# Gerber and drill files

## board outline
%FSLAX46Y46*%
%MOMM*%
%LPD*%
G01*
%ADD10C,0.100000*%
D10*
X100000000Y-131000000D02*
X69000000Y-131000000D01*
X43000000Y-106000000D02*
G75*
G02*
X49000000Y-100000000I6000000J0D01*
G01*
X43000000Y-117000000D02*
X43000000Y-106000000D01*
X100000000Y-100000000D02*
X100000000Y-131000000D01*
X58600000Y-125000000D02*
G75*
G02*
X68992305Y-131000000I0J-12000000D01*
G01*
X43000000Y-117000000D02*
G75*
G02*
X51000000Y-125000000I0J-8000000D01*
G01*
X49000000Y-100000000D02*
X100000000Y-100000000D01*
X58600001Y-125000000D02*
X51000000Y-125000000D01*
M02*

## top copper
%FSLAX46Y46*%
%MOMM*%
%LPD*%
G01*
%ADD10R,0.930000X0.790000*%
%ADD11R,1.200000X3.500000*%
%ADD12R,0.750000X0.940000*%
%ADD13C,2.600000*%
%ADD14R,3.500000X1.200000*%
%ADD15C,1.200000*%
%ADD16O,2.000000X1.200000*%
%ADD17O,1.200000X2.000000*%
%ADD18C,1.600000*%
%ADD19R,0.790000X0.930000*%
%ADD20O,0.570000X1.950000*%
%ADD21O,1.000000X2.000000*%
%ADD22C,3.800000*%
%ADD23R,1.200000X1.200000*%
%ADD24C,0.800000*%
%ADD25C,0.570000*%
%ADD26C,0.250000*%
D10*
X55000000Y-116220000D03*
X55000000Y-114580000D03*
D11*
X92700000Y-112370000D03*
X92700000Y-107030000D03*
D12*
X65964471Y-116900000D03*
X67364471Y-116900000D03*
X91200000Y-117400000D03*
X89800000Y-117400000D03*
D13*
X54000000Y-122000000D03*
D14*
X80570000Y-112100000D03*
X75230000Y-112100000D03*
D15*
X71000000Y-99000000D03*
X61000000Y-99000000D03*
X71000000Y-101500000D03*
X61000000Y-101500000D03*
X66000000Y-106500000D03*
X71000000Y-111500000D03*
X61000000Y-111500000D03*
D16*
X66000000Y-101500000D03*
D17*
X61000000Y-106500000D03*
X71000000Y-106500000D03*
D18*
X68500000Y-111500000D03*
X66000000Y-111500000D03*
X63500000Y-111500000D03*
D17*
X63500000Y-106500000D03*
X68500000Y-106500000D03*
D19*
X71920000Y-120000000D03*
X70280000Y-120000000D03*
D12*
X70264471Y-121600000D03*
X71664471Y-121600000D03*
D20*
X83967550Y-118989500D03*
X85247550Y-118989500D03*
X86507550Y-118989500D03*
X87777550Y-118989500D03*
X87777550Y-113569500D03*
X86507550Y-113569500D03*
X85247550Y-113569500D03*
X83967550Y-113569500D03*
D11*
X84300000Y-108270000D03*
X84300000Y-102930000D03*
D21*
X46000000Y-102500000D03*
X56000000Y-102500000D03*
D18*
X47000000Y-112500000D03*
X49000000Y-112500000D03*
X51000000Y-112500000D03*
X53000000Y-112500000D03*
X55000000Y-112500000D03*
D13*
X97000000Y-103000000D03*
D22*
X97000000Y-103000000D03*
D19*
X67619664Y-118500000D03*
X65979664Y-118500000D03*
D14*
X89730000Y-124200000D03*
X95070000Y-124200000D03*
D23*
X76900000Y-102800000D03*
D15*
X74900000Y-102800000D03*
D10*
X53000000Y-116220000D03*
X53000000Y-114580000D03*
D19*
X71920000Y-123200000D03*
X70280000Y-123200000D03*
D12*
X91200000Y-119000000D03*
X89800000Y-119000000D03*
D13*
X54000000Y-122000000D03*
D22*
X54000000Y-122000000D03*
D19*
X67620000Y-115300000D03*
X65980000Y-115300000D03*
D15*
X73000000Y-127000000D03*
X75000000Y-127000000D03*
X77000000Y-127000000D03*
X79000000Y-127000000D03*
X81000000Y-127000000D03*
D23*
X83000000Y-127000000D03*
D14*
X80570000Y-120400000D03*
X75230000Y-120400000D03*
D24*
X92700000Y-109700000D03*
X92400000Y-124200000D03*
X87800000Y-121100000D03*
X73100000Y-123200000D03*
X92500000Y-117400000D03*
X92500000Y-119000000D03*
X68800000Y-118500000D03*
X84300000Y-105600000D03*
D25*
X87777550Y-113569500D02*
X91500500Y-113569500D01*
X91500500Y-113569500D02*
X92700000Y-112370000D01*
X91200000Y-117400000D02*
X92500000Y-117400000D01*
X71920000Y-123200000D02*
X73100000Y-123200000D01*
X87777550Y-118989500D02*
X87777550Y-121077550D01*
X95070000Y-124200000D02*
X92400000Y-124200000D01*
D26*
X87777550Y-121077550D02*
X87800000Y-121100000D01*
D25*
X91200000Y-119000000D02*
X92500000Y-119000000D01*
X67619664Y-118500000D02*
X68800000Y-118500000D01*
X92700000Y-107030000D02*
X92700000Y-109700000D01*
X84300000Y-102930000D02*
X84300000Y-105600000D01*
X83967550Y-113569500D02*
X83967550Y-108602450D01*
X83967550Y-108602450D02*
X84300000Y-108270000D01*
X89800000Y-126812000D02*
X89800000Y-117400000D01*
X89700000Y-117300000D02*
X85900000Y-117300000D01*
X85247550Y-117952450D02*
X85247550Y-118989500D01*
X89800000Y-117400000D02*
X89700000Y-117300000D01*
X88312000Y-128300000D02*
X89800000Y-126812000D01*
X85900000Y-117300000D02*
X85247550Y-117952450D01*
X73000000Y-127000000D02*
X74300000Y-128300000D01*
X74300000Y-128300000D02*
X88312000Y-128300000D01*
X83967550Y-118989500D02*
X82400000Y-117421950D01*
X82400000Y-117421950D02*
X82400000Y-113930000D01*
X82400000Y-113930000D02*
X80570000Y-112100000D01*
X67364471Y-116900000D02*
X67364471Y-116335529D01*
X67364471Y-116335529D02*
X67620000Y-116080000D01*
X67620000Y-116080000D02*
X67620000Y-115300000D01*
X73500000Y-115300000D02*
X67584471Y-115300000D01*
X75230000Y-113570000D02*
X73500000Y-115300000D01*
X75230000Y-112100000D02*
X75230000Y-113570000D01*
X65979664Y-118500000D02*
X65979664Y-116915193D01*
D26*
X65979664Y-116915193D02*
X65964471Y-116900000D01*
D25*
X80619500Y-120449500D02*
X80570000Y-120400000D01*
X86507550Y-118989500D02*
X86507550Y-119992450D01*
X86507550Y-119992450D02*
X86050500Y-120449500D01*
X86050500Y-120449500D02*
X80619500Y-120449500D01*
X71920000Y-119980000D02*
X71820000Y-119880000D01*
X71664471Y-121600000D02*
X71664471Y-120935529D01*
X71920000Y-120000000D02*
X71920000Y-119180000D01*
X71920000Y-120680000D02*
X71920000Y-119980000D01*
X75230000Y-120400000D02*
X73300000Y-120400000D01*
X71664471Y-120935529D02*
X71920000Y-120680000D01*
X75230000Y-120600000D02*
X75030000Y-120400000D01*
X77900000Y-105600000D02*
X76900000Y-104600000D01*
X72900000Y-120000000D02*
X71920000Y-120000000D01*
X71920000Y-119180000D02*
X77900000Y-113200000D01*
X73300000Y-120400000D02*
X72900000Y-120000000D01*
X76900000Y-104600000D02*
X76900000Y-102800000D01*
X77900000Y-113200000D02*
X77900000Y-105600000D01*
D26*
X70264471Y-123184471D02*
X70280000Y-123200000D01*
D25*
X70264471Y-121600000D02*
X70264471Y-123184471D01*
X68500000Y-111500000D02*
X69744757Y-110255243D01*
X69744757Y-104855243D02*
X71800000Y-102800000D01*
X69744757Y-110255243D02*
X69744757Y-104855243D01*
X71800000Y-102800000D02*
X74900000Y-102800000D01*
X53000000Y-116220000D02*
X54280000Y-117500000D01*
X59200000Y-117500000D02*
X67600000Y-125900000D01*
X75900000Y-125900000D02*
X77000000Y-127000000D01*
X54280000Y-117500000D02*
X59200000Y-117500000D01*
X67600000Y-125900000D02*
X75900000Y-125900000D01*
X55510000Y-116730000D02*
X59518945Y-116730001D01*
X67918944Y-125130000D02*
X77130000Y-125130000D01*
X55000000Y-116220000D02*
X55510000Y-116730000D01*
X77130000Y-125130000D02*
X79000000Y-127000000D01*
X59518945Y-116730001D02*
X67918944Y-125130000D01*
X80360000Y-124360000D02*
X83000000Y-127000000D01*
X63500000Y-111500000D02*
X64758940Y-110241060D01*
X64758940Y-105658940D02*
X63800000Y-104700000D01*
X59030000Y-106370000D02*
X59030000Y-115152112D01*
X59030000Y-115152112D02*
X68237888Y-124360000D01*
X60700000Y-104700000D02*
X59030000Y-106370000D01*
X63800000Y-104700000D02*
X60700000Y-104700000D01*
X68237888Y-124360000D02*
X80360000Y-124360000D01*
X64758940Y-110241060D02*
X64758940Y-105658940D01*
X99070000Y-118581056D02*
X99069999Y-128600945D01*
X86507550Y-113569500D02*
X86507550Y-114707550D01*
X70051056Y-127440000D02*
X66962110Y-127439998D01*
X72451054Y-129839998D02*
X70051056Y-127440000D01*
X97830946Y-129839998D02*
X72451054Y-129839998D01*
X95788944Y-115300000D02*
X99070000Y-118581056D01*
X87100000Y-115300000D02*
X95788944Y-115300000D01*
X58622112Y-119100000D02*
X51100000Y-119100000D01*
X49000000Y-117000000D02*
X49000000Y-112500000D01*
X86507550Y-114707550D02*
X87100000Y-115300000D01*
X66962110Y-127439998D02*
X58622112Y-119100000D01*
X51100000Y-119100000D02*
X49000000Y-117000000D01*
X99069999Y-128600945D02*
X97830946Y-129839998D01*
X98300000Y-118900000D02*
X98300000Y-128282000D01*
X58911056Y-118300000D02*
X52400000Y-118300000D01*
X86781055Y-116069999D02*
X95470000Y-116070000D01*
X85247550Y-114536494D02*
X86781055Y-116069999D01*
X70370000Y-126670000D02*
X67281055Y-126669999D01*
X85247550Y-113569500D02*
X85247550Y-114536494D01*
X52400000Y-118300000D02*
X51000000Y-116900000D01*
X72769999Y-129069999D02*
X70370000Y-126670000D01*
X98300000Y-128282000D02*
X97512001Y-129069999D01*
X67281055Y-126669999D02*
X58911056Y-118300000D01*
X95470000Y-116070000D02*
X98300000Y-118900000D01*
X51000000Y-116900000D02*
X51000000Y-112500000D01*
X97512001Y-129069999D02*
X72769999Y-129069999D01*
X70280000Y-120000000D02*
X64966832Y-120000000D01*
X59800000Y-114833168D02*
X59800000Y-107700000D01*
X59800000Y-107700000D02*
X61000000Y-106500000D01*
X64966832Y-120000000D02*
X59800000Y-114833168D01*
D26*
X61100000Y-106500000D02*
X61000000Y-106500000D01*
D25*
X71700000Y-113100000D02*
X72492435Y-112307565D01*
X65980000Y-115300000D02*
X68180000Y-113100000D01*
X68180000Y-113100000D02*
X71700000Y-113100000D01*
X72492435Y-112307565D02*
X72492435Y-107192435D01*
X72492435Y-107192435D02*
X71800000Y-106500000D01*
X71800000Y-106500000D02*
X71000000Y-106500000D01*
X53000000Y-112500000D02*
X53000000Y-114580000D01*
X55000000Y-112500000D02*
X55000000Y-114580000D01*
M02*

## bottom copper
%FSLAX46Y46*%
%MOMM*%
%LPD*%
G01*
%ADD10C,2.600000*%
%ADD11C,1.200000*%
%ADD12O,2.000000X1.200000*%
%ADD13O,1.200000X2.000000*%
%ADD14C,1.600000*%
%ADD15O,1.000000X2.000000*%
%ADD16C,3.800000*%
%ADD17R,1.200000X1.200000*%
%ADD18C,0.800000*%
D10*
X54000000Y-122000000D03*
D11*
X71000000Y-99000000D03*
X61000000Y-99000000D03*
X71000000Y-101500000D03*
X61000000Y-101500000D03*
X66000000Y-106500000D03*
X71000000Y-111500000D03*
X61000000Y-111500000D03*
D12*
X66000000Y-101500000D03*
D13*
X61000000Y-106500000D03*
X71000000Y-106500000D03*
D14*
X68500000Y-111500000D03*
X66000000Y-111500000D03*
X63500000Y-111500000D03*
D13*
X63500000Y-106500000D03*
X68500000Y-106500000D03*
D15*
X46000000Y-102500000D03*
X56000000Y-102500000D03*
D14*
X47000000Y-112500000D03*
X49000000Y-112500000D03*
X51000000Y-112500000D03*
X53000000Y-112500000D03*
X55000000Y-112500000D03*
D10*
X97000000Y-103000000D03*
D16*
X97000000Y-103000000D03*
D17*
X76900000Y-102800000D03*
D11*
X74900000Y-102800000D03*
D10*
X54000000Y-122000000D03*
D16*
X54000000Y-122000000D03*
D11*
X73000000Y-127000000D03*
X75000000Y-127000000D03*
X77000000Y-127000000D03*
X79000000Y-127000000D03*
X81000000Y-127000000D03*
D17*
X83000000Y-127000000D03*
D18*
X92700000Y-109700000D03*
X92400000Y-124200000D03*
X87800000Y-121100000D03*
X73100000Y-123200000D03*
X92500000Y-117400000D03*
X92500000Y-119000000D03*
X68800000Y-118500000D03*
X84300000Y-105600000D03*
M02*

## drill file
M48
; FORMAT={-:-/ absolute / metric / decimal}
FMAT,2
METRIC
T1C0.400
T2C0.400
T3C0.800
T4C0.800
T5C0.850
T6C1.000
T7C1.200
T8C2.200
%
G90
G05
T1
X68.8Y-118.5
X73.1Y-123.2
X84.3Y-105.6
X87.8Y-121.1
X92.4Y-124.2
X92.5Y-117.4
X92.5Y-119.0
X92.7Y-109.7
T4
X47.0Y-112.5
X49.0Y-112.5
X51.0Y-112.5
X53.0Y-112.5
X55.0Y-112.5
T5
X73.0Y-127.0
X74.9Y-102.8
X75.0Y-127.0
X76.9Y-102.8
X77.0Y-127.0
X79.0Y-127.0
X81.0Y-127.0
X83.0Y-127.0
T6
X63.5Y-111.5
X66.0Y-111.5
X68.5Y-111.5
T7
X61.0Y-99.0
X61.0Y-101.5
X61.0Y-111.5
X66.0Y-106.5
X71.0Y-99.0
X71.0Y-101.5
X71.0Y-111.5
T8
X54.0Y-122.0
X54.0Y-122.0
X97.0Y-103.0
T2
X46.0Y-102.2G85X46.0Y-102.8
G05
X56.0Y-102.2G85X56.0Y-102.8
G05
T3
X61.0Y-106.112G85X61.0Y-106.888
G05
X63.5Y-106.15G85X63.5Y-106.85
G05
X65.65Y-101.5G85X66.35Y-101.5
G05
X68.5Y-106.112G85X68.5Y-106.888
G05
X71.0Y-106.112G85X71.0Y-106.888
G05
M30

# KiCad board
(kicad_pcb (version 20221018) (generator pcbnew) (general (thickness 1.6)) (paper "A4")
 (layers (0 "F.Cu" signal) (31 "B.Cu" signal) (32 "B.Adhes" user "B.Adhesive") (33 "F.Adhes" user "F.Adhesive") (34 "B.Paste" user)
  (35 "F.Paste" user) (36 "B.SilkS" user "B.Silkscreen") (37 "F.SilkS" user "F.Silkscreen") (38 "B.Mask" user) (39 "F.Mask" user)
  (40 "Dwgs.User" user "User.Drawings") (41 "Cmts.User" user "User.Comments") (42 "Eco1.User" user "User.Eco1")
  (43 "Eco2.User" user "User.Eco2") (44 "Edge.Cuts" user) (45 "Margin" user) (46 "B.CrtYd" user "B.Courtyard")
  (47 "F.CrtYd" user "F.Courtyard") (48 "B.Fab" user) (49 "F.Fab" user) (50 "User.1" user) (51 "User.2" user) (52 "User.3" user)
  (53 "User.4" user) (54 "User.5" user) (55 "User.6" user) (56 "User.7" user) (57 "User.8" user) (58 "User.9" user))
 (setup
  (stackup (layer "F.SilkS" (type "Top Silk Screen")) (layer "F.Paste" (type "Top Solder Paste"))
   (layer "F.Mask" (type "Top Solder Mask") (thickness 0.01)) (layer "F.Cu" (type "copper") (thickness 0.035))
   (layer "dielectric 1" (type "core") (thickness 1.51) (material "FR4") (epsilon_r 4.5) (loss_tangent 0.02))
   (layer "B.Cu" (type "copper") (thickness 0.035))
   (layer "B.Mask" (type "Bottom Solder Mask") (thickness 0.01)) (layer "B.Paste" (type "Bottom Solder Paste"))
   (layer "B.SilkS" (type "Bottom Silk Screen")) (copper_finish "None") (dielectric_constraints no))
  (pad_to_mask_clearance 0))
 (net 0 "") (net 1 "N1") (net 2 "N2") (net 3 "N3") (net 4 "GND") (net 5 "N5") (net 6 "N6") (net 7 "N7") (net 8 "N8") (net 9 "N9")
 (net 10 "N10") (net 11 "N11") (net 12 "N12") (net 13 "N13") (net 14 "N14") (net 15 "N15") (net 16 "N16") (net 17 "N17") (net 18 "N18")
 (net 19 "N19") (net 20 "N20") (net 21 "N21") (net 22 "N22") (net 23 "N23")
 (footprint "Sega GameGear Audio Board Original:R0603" (layer "F.Cu") (at 55 115.4 90)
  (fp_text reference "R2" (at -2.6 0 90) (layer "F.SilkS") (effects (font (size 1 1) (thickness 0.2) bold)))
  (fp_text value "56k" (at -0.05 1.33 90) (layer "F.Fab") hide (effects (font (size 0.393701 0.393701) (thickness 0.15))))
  (pad "1" smd rect (at -0.82 0 90) (size 0.79 0.93) (layers "F.Cu" "F.Paste" "F.Mask") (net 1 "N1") (solder_mask_margin 0.102))
  (pad "2" smd rect (at 0.82 0 90) (size 0.79 0.93) (layers "F.Cu" "F.Paste" "F.Mask") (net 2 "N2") (solder_mask_margin 0.102)))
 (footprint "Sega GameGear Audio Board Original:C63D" (layer "F.Cu") (at 92.7 109.7 90)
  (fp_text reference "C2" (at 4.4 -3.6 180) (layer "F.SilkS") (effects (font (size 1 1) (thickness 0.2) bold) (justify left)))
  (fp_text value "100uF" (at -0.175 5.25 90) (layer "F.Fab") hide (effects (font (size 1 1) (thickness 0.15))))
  (pad "1" smd rect (at -2.67 0 90) (size 3.5 1.2) (layers "F.Cu" "F.Paste" "F.Mask") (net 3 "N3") (solder_mask_margin 0.102))
  (pad "2" smd rect (at 2.67 0 90) (size 3.5 1.2) (layers "F.Cu" "F.Paste" "F.Mask") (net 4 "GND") (solder_mask_margin 0.102)))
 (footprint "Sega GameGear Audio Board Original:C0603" (layer "F.Cu") (at 66.664471 116.9)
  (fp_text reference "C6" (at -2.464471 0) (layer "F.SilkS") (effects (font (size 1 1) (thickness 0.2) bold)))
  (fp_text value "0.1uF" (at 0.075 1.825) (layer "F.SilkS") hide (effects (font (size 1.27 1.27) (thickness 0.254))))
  (pad "1" smd rect (at -0.7 0) (size 0.75 0.94) (layers "F.Cu" "F.Paste" "F.Mask") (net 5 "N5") (solder_mask_margin 0.102))
  (pad "2" smd rect (at 0.7 0) (size 0.75 0.94) (layers "F.Cu" "F.Paste" "F.Mask") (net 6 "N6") (solder_mask_margin 0.102)))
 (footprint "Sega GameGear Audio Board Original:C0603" (layer "F.Cu") (at 90.5 117.4 180)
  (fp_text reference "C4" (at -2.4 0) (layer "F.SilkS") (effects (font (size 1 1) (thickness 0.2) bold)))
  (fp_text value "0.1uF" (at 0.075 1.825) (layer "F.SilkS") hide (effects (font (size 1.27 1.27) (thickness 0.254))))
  (pad "1" smd rect (at -0.7 0 180) (size 0.75 0.94) (layers "F.Cu" "F.Paste" "F.Mask") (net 4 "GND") (solder_mask_margin 0.102))
  (pad "2" smd rect (at 0.7 0 180) (size 0.75 0.94) (layers "F.Cu" "F.Paste" "F.Mask") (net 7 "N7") (solder_mask_margin 0.102)))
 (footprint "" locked (layer "F.Cu") (at 54 122)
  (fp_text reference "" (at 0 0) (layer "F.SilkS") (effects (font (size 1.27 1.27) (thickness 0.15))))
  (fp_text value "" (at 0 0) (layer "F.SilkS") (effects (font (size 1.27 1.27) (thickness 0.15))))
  (pad "1" thru_hole circle locked (at 0 0) (size 2.6 2.6) (drill 2.2) (layers "*.Cu" "*.Mask")))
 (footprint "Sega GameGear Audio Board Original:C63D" (layer "F.Cu") (at 77.9 112.1 180)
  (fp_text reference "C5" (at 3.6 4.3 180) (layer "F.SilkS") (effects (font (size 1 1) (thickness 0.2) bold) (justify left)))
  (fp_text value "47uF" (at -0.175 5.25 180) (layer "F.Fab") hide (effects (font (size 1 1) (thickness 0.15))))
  (pad "1" smd rect (at -2.67 0 180) (size 3.5 1.2) (layers "F.Cu" "F.Paste" "F.Mask") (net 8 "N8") (solder_mask_margin 0.102))
  (pad "2" smd rect (at 2.67 0 180) (size 3.5 1.2) (layers "F.Cu" "F.Paste" "F.Mask") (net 6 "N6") (solder_mask_margin 0.102)))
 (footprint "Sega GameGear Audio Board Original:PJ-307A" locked (layer "F.Cu") (at 66 106.5 -90)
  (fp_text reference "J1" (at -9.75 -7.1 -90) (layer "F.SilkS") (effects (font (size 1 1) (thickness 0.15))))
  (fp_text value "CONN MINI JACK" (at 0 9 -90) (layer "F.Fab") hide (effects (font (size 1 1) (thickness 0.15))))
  (pad "" thru_hole circle locked (at -7.5 -5 270) (size 1.2 1.2) (drill 1.2) (layers "*.Cu" "*.Mask"))
  (pad "" thru_hole circle locked (at -7.5 5 270) (size 1.2 1.2) (drill 1.2) (layers "*.Cu" "*.Mask"))
  (pad "" thru_hole circle locked (at -5 -5 270) (size 1.2 1.2) (drill 1.2) (layers "*.Cu" "*.Mask"))
  (pad "" thru_hole circle locked (at -5 5 270) (size 1.2 1.2) (drill 1.2) (layers "*.Cu" "*.Mask"))
  (pad "" thru_hole circle locked (at 0 0 270) (size 1.2 1.2) (drill 1.2) (layers "*.Cu" "*.Mask"))
  (pad "" thru_hole circle locked (at 5 -5 270) (size 1.2 1.2) (drill 1.2) (layers "*.Cu" "*.Mask"))
  (pad "" thru_hole circle locked (at 5 5 270) (size 1.2 1.2) (drill 1.2) (layers "*.Cu" "*.Mask"))
  (pad "1" thru_hole oval locked (at -5 0) (size 2 1.2) (drill oval 1.499997 0.799998) (layers "*.Cu" "*.Mask") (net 4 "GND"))
  (pad "2" thru_hole oval locked (at 0 5 270) (size 2 1.2) (drill oval 1.575029 0.799998) (layers "*.Cu" "*.Mask") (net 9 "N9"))
  (pad "3" thru_hole oval locked (at 0 -5 270) (size 2 1.2) (drill oval 1.575029 0.799998) (layers "*.Cu" "*.Mask") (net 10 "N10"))
  (pad "4" thru_hole circle locked (at 5 -2.5 270) (size 1.6 1.6) (drill 0.999998) (layers "*.Cu" "*.Mask") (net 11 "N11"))
  (pad "5" thru_hole circle locked (at 5 0 270) (size 1.6 1.6) (drill 0.999998) (layers "*.Cu" "*.Mask") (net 4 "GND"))
  (pad "6" thru_hole circle locked (at 5 2.5 270) (size 1.6 1.6) (drill 0.999998) (layers "*.Cu" "*.Mask") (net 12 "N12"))
  (pad "10" thru_hole oval locked (at 0 2.5 270) (size 2 1.2) (drill oval 1.499997 0.799998) (layers "*.Cu" "*.Mask") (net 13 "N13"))
  (pad "11" thru_hole oval locked (at 0 -2.5 270) (size 2 1.2) (drill oval 1.575029 0.799998) (layers "*.Cu" "*.Mask") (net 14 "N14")))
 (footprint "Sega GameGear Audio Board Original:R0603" (layer "F.Cu") (at 71.1 120 180)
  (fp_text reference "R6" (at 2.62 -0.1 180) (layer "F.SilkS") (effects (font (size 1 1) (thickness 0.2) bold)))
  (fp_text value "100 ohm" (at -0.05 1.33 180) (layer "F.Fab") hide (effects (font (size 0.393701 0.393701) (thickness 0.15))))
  (pad "1" smd rect (at -0.82 0 180) (size 0.79 0.93) (layers "F.Cu" "F.Paste" "F.Mask") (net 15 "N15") (solder_mask_margin 0.102))
  (pad "2" smd rect (at 0.82 0 180) (size 0.79 0.93) (layers "F.Cu" "F.Paste" "F.Mask") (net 9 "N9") (solder_mask_margin 0.102)))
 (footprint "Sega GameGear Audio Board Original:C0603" (layer "F.Cu") (at 70.964471 121.6)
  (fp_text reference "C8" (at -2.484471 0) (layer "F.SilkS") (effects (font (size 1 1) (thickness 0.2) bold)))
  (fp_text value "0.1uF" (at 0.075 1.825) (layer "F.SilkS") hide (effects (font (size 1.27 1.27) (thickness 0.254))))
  (pad "1" smd rect (at -0.7 0) (size 0.75 0.94) (layers "F.Cu" "F.Paste" "F.Mask") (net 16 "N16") (solder_mask_margin 0.102))
  (pad "2" smd rect (at 0.7 0) (size 0.75 0.94) (layers "F.Cu" "F.Paste" "F.Mask") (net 15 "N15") (solder_mask_margin 0.102)))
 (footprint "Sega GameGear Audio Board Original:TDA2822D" (layer "F.Cu") (at 85.88255 116.3 90)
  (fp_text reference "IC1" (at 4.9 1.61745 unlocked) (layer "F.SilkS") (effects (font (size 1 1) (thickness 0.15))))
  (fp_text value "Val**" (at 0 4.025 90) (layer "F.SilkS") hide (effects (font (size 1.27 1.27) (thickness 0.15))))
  (pad "1" smd oval (at -2.6895 -1.915) (size 0.57 1.95) (layers "F.Cu" "F.Paste" "F.Mask") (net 8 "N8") (solder_mask_margin 0.102))
  (pad "2" smd oval (at -2.6895 -0.635) (size 0.57 1.95) (layers "F.Cu" "F.Paste" "F.Mask") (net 7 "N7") (solder_mask_margin 0.102))
  (pad "3" smd oval (at -2.6895 0.625) (size 0.57 1.95) (layers "F.Cu" "F.Paste" "F.Mask") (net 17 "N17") (solder_mask_margin 0.102))
  (pad "4" smd oval (at -2.6895 1.895) (size 0.57 1.95) (layers "F.Cu" "F.Paste" "F.Mask") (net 4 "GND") (solder_mask_margin 0.102))
  (pad "5" smd oval (at 2.7305 1.895) (size 0.57 1.95) (layers "F.Cu" "F.Paste" "F.Mask") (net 3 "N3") (solder_mask_margin 0.102))
  (pad "6" smd oval (at 2.7305 0.625) (size 0.57 1.95) (layers "F.Cu" "F.Paste" "F.Mask") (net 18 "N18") (solder_mask_margin 0.102))
  (pad "7" smd oval (at 2.7305 -0.635) (size 0.57 1.95) (layers "F.Cu" "F.Paste" "F.Mask") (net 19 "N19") (solder_mask_margin 0.102))
  (pad "8" smd oval (at 2.7305 -1.915) (size 0.57 1.95) (layers "F.Cu" "F.Paste" "F.Mask") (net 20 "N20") (solder_mask_margin 0.102)))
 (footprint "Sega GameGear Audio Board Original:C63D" (layer "F.Cu") (at 84.3 105.6 90)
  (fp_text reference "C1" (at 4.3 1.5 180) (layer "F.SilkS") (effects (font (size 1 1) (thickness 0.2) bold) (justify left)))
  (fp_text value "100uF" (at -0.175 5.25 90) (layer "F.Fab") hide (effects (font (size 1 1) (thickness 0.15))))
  (pad "1" smd rect (at -2.67 0 90) (size 3.5 1.2) (layers "F.Cu" "F.Paste" "F.Mask") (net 20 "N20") (solder_mask_margin 0.102))
  (pad "2" smd rect (at 2.67 0 90) (size 3.5 1.2) (layers "F.Cu" "F.Paste" "F.Mask") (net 4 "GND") (solder_mask_margin 0.102)))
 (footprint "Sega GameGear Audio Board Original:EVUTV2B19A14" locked (layer "F.Cu") (at 51 102.5)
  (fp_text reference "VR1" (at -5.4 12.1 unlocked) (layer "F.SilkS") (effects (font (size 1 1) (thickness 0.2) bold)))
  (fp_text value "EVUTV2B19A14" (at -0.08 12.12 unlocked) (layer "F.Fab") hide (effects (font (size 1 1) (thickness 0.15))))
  (pad "" thru_hole oval locked (at -5 0) (size 1 2) (drill oval 0.4 1) (layers "*.Cu" "*.Mask"))
  (pad "" thru_hole oval locked (at 5 0) (size 1 2) (drill oval 0.4 1) (layers "*.Cu" "*.Mask"))
  (pad "1" thru_hole circle locked (at -4 10) (size 1.6 1.6) (drill 0.8) (layers "*.Cu" "*.Mask") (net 4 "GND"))
  (pad "2" thru_hole circle locked (at -2 10) (size 1.6 1.6) (drill 0.8) (layers "*.Cu" "*.Mask") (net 18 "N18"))
  (pad "3" thru_hole circle locked (at 0 10) (size 1.6 1.6) (drill 0.8) (layers "*.Cu" "*.Mask") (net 19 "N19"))
  (pad "4" thru_hole circle locked (at 2 10) (size 1.6 1.6) (drill 0.8) (layers "*.Cu" "*.Mask") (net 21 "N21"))
  (pad "5" thru_hole circle locked (at 4 10) (size 1.6 1.6) (drill 0.8) (layers "*.Cu" "*.Mask") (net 2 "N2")))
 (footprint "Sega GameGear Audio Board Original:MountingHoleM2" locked (layer "F.Cu") (at 97 103)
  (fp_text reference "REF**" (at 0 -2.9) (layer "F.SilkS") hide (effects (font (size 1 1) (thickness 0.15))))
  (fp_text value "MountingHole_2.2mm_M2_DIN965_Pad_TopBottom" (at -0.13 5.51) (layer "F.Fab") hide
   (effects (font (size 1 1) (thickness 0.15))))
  (pad "1" thru_hole circle locked (at 0 0) (size 2.6 2.6) (drill 2.2) (layers "*.Cu" "*.Mask"))
  (pad "1" connect circle locked (at 0 0) (size 3.8 3.8) (layers "F.Cu" "F.Mask"))
  (pad "1" connect circle locked (at 0 0) (size 3.8 3.8) (layers "B.Cu" "B.Mask")))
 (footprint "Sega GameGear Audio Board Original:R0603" (layer "F.Cu") (at 66.799664 118.5 180)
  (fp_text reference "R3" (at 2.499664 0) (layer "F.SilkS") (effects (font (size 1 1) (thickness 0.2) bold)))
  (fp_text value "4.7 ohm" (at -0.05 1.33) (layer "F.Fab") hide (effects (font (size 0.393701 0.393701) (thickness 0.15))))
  (pad "1" smd rect (at -0.82 0 180) (size 0.79 0.93) (layers "F.Cu" "F.Paste" "F.Mask") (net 4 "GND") (solder_mask_margin 0.102))
  (pad "2" smd rect (at 0.82 0 180) (size 0.79 0.93) (layers "F.Cu" "F.Paste" "F.Mask") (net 5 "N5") (solder_mask_margin 0.102)))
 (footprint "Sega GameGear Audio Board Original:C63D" (layer "F.Cu") (at 92.4 124.2)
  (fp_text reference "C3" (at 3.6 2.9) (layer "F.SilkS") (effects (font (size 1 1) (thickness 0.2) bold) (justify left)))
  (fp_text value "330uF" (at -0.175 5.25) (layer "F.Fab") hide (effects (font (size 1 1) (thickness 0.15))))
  (pad "1" smd rect (at -2.67 0) (size 3.5 1.2) (layers "F.Cu" "F.Paste" "F.Mask") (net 7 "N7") (solder_mask_margin 0.102))
  (pad "2" smd rect (at 2.67 0) (size 3.5 1.2) (layers "F.Cu" "F.Paste" "F.Mask") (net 4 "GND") (solder_mask_margin 0.102)))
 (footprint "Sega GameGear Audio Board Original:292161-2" (layer "F.Cu") (at 76.9 102.8)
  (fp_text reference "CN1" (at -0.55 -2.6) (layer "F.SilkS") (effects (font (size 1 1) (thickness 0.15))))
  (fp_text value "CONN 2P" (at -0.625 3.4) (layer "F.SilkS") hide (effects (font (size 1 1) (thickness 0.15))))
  (pad "1" thru_hole rect (at 0 0) (size 1.2 1.2) (drill 0.85) (layers "*.Cu" "*.Mask") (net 15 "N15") (solder_mask_margin 0.102))
  (pad "2" thru_hole circle (at -2 0) (size 1.2 1.2) (drill 0.85) (layers "*.Cu" "*.Mask") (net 11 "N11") (solder_mask_margin 0.102)))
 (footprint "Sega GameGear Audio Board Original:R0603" (layer "F.Cu") (at 53 115.4 90)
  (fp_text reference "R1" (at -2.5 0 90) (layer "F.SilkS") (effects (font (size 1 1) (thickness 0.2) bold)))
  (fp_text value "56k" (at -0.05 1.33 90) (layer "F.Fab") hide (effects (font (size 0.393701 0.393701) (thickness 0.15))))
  (pad "1" smd rect (at -0.82 0 90) (size 0.79 0.93) (layers "F.Cu" "F.Paste" "F.Mask") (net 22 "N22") (solder_mask_margin 0.102))
  (pad "2" smd rect (at 0.82 0 90) (size 0.79 0.93) (layers "F.Cu" "F.Paste" "F.Mask") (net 21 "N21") (solder_mask_margin 0.102)))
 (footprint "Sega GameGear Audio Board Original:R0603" (layer "F.Cu") (at 71.1 123.2 180)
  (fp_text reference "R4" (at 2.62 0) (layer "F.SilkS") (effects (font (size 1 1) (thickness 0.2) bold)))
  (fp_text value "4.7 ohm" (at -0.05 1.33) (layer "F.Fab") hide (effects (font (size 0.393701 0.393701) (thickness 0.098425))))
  (pad "1" smd rect (at -0.82 0 180) (size 0.79 0.93) (layers "F.Cu" "F.Paste" "F.Mask") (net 4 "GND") (solder_mask_margin 0.102))
  (pad "2" smd rect (at 0.82 0 180) (size 0.79 0.93) (layers "F.Cu" "F.Paste" "F.Mask") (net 16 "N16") (solder_mask_margin 0.102)))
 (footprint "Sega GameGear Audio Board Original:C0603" (layer "F.Cu") (at 90.5 119 180)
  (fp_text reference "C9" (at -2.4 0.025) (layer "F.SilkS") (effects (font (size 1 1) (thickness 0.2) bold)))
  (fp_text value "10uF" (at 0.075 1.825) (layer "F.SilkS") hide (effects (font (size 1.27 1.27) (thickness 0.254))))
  (pad "1" smd rect (at -0.7 0 180) (size 0.75 0.94) (layers "F.Cu" "F.Paste" "F.Mask") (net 4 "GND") (solder_mask_margin 0.102))
  (pad "2" smd rect (at 0.7 0 180) (size 0.75 0.94) (layers "F.Cu" "F.Paste" "F.Mask") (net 7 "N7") (solder_mask_margin 0.102)))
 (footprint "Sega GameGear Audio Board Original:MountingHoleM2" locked (layer "F.Cu") (at 54 122)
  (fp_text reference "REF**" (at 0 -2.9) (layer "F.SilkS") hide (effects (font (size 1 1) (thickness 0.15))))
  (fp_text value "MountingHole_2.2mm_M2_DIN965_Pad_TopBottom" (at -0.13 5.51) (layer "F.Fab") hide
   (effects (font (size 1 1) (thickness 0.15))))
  (pad "1" thru_hole circle locked (at 0 0) (size 2.6 2.6) (drill 2.2) (layers "*.Cu" "*.Mask"))
  (pad "1" connect circle locked (at 0 0) (size 3.8 3.8) (layers "F.Cu" "F.Mask"))
  (pad "1" connect circle locked (at 0 0) (size 3.8 3.8) (layers "B.Cu" "B.Mask")))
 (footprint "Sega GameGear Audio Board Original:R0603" (layer "F.Cu") (at 66.8 115.3 180)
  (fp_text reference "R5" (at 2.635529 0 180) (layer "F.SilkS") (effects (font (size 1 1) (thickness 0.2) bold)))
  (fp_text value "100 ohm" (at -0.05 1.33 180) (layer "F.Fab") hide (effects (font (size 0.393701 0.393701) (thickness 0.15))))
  (pad "1" smd rect (at -0.82 0 180) (size 0.79 0.93) (layers "F.Cu" "F.Paste" "F.Mask") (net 6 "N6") (solder_mask_margin 0.102))
  (pad "2" smd rect (at 0.82 0 180) (size 0.79 0.93) (layers "F.Cu" "F.Paste" "F.Mask") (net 10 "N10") (solder_mask_margin 0.102)))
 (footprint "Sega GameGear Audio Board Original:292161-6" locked (layer "F.Cu") (at 83 127)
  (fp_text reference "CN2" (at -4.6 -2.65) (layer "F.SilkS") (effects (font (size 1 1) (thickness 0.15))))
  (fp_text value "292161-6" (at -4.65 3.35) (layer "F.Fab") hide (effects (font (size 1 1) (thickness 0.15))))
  (pad "1" thru_hole circle locked (at -10 0) (size 1.2 1.2) (drill 0.85) (layers "*.Cu" "*.Mask") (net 7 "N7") (solder_mask_margin 0.102))
  (pad "2" thru_hole circle locked (at -8 0) (size 1.2 1.2) (drill 0.85) (layers "*.Cu" "*.Mask") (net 4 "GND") (solder_mask_margin 0.102))
  (pad "3" thru_hole circle locked (at -6 0) (size 1.2 1.2) (drill 0.85) (layers "*.Cu" "*.Mask") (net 22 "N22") (solder_mask_margin 0.102))
  (pad "4" thru_hole circle locked (at -4 0) (size 1.2 1.2) (drill 0.85) (layers "*.Cu" "*.Mask") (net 1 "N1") (solder_mask_margin 0.102))
  (pad "5" thru_hole circle locked (at -2 0) (size 1.2 1.2) (drill 0.85) (layers "*.Cu" "*.Mask") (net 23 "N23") (solder_mask_margin 0.102))
  (pad "6" thru_hole rect locked (at 0 0) (size 1.2 1.2) (drill 0.85) (layers "*.Cu" "*.Mask") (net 12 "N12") (solder_mask_margin 0.102)))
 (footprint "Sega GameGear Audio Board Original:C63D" (layer "F.Cu") (at 77.9 120.4 180)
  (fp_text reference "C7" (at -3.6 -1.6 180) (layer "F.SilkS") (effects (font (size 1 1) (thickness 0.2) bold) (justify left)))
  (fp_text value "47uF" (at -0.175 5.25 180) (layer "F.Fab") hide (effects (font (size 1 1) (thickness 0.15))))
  (pad "1" smd rect (at -2.67 0 180) (size 3.5 1.2) (layers "F.Cu" "F.Paste" "F.Mask") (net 17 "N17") (solder_mask_margin 0.102))
  (pad "2" smd rect (at 2.67 0 180) (size 3.5 1.2) (layers "F.Cu" "F.Paste" "F.Mask") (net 15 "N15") (solder_mask_margin 0.102)))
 (gr_line locked (start 100 131) (end 69 131) (stroke (width 0.1) (type solid)) (layer "Edge.Cuts"))
 (gr_arc locked (start 43 106) (mid 44.757359 101.757359) (end 49 100) (stroke (width 0.1) (type solid)) (layer "Edge.Cuts"))
 (gr_line locked (start 43 117) (end 43 106) (stroke (width 0.1) (type solid)) (layer "Edge.Cuts"))
 (gr_line locked (start 100 100) (end 100 131) (stroke (width 0.1) (type solid)) (layer "Edge.Cuts"))
 (gr_arc locked (start 58.6 125) (mid 64.6 126.607695) (end 68.992305 131) (stroke (width 0.1) (type solid)) (layer "Edge.Cuts"))
 (gr_arc locked (start 43 117) (mid 48.656854 119.343146) (end 51 125) (stroke (width 0.1) (type solid)) (layer "Edge.Cuts"))
 (gr_line locked (start 49 100) (end 100 100) (stroke (width 0.1) (type solid)) (layer "Edge.Cuts"))
 (gr_line locked (start 58.600001 125) (end 51 125) (stroke (width 0.1) (type solid)) (layer "Edge.Cuts"))
 (segment (start 87.77755 113.5695) (end 91.5005 113.5695) (width 0.57) (layer "F.Cu") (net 3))
 (segment (start 91.5005 113.5695) (end 92.7 112.37) (width 0.57) (layer "F.Cu") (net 3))
 (segment (start 91.2 117.4) (end 92.5 117.4) (width 0.57) (layer "F.Cu") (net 4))
 (segment (start 71.92 123.2) (end 73.1 123.2) (width 0.57) (layer "F.Cu") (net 4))
 (segment (start 87.77755 118.9895) (end 87.77755 121.07755) (width 0.57) (layer "F.Cu") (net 4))
 (segment (start 95.07 124.2) (end 92.4 124.2) (width 0.57) (layer "F.Cu") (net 4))
 (segment (start 87.77755 121.07755) (end 87.8 121.1) (width 0.25) (layer "F.Cu") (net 4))
 (segment (start 91.2 119) (end 92.5 119) (width 0.57) (layer "F.Cu") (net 4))
 (segment (start 67.619664 118.5) (end 68.8 118.5) (width 0.57) (layer "F.Cu") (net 4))
 (segment (start 92.7 107.03) (end 92.7 109.7) (width 0.57) (layer "F.Cu") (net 4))
 (segment (start 84.3 102.93) (end 84.3 105.6) (width 0.57) (layer "F.Cu") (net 4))
 (via (at 92.7 109.7) (size 0.8) (drill 0.4) (layers "F.Cu" "B.Cu") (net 4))
 (via (at 92.4 124.2) (size 0.8) (drill 0.4) (layers "F.Cu" "B.Cu") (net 4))
 (via (at 87.8 121.1) (size 0.8) (drill 0.4) (layers "F.Cu" "B.Cu") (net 4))
 (via (at 73.1 123.2) (size 0.8) (drill 0.4) (layers "F.Cu" "B.Cu") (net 4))
 (via (at 92.5 117.4) (size 0.8) (drill 0.4) (layers "F.Cu" "B.Cu") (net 4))
 (via (at 92.5 119) (size 0.8) (drill 0.4) (layers "F.Cu" "B.Cu") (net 4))
 (via (at 68.8 118.5) (size 0.8) (drill 0.4) (layers "F.Cu" "B.Cu") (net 4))
 (via (at 84.3 105.6) (size 0.8) (drill 0.4) (layers "F.Cu" "B.Cu") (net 4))
 (segment (start 83.96755 113.5695) (end 83.96755 108.60245) (width 0.57) (layer "F.Cu") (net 20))
 (segment (start 83.96755 108.60245) (end 84.3 108.27) (width 0.57) (layer "F.Cu") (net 20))
 (segment (start 89.8 126.812) (end 89.8 117.4) (width 0.57) (layer "F.Cu") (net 7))
 (segment (start 89.7 117.3) (end 85.9 117.3) (width 0.57) (layer "F.Cu") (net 7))
 (segment (start 85.24755 117.95245) (end 85.24755 118.9895) (width 0.57) (layer "F.Cu") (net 7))
 (segment (start 89.8 117.4) (end 89.7 117.3) (width 0.57) (layer "F.Cu") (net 7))
 (segment (start 88.312 128.3) (end 89.8 126.812) (width 0.57) (layer "F.Cu") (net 7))
 (segment (start 85.9 117.3) (end 85.24755 117.95245) (width 0.57) (layer "F.Cu") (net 7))
 (segment (start 73 127) (end 74.3 128.3) (width 0.57) (layer "F.Cu") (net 7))
 (segment (start 74.3 128.3) (end 88.312 128.3) (width 0.57) (layer "F.Cu") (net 7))
 (segment (start 83.96755 118.9895) (end 82.4 117.42195) (width 0.57) (layer "F.Cu") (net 8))
 (segment (start 82.4 117.42195) (end 82.4 113.93) (width 0.57) (layer "F.Cu") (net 8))
 (segment (start 82.4 113.93) (end 80.57 112.1) (width 0.57) (layer "F.Cu") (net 8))
 (segment (start 67.364471 116.9) (end 67.364471 116.335529) (width 0.57) (layer "F.Cu") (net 6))
 (segment (start 67.364471 116.335529) (end 67.62 116.08) (width 0.57) (layer "F.Cu") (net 6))
 (segment (start 67.62 116.08) (end 67.62 115.3) (width 0.57) (layer "F.Cu") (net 6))
 (segment (start 73.5 115.3) (end 67.584471 115.3) (width 0.57) (layer "F.Cu") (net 6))
 (segment (start 75.23 113.57) (end 73.5 115.3) (width 0.57) (layer "F.Cu") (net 6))
 (segment (start 75.23 112.1) (end 75.23 113.57) (width 0.57) (layer "F.Cu") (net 6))
 (segment (start 65.979664 118.5) (end 65.979664 116.915193) (width 0.57) (layer "F.Cu") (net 5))
 (segment (start 65.979664 116.915193) (end 65.964471 116.9) (width 0.25) (layer "F.Cu") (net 5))
 (segment (start 80.6195 120.4495) (end 80.57 120.4) (width 0.57) (layer "F.Cu") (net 17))
 (segment (start 86.50755 118.9895) (end 86.50755 119.99245) (width 0.57) (layer "F.Cu") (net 17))
 (segment (start 86.50755 119.99245) (end 86.0505 120.4495) (width 0.57) (layer "F.Cu") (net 17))
 (segment (start 86.0505 120.4495) (end 80.6195 120.4495) (width 0.57) (layer "F.Cu") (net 17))
 (segment (start 71.92 119.98) (end 71.82 119.88) (width 0.57) (layer "F.Cu") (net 15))
 (segment (start 71.664471 121.6) (end 71.664471 120.935529) (width 0.57) (layer "F.Cu") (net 15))
 (segment (start 71.92 120) (end 71.92 119.18) (width 0.57) (layer "F.Cu") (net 15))
 (segment (start 71.92 120.68) (end 71.92 119.98) (width 0.57) (layer "F.Cu") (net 15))
 (segment (start 75.23 120.4) (end 73.3 120.4) (width 0.57) (layer "F.Cu") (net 15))
 (segment (start 71.664471 120.935529) (end 71.92 120.68) (width 0.57) (layer "F.Cu") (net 15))
 (segment (start 75.23 120.6) (end 75.03 120.4) (width 0.57) (layer "F.Cu") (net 15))
 (segment (start 77.9 105.6) (end 76.9 104.6) (width 0.57) (layer "F.Cu") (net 15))
 (segment (start 72.9 120) (end 71.92 120) (width 0.57) (layer "F.Cu") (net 15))
 (segment (start 71.92 119.18) (end 77.9 113.2) (width 0.57) (layer "F.Cu") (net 15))
 (segment (start 73.3 120.4) (end 72.9 120) (width 0.57) (layer "F.Cu") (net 15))
 (segment (start 76.9 104.6) (end 76.9 102.8) (width 0.57) (layer "F.Cu") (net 15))
 (segment (start 77.9 113.2) (end 77.9 105.6) (width 0.57) (layer "F.Cu") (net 15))
 (segment (start 70.264471 123.184471) (end 70.28 123.2) (width 0.25) (layer "F.Cu") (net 16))
 (segment (start 70.264471 121.6) (end 70.264471 123.184471) (width 0.57) (layer "F.Cu") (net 16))
 (segment (start 68.5 111.5) (end 69.744757 110.255243) (width 0.57) (layer "F.Cu") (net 11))
 (segment (start 69.744757 104.855243) (end 71.8 102.8) (width 0.57) (layer "F.Cu") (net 11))
 (segment (start 69.744757 110.255243) (end 69.744757 104.855243) (width 0.57) (layer "F.Cu") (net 11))
 (segment (start 71.8 102.8) (end 74.9 102.8) (width 0.57) (layer "F.Cu") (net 11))
 (segment (start 53 116.22) (end 54.28 117.5) (width 0.57) (layer "F.Cu") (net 22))
 (segment (start 59.2 117.5) (end 67.6 125.9) (width 0.57) (layer "F.Cu") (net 22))
 (segment (start 75.9 125.9) (end 77 127) (width 0.57) (layer "F.Cu") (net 22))
 (segment (start 54.28 117.5) (end 59.2 117.5) (width 0.57) (layer "F.Cu") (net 22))
 (segment (start 67.6 125.9) (end 75.9 125.9) (width 0.57) (layer "F.Cu") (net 22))
 (segment (start 55.51 116.73) (end 59.518945 116.730001) (width 0.57) (layer "F.Cu") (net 1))
 (segment (start 67.918944 125.13) (end 77.13 125.13) (width 0.57) (layer "F.Cu") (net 1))
 (segment (start 55 116.22) (end 55.51 116.73) (width 0.57) (layer "F.Cu") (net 1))
 (segment (start 77.13 125.13) (end 79 127) (width 0.57) (layer "F.Cu") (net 1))
 (segment (start 59.518945 116.730001) (end 67.918944 125.13) (width 0.57) (layer "F.Cu") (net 1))
 (segment (start 80.36 124.36) (end 83 127) (width 0.57) (layer "F.Cu") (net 12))
 (segment (start 63.5 111.5) (end 64.75894 110.24106) (width 0.57) (layer "F.Cu") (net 12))
 (segment (start 64.75894 105.65894) (end 63.8 104.7) (width 0.57) (layer "F.Cu") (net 12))
 (segment (start 59.03 106.37) (end 59.03 115.152112) (width 0.57) (layer "F.Cu") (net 12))
 (segment (start 59.03 115.152112) (end 68.237888 124.36) (width 0.57) (layer "F.Cu") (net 12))
 (segment (start 60.7 104.7) (end 59.03 106.37) (width 0.57) (layer "F.Cu") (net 12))
 (segment (start 63.8 104.7) (end 60.7 104.7) (width 0.57) (layer "F.Cu") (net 12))
 (segment (start 68.237888 124.36) (end 80.36 124.36) (width 0.57) (layer "F.Cu") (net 12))
 (segment (start 64.75894 110.24106) (end 64.75894 105.65894) (width 0.57) (layer "F.Cu") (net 12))
 (segment (start 99.07 118.581056) (end 99.069999 128.600945) (width 0.57) (layer "F.Cu") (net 18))
 (segment (start 86.50755 113.5695) (end 86.50755 114.70755) (width 0.57) (layer "F.Cu") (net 18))
 (segment (start 70.051056 127.44) (end 66.96211 127.439998) (width 0.57) (layer "F.Cu") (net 18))
 (segment (start 72.451054 129.839998) (end 70.051056 127.44) (width 0.57) (layer "F.Cu") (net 18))
 (segment (start 97.830946 129.839998) (end 72.451054 129.839998) (width 0.57) (layer "F.Cu") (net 18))
 (segment (start 95.788944 115.3) (end 99.07 118.581056) (width 0.57) (layer "F.Cu") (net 18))
 (segment (start 87.1 115.3) (end 95.788944 115.3) (width 0.57) (layer "F.Cu") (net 18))
 (segment (start 58.622112 119.1) (end 51.1 119.1) (width 0.57) (layer "F.Cu") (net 18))
 (segment (start 49 117) (end 49 112.5) (width 0.57) (layer "F.Cu") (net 18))
 (segment (start 86.50755 114.70755) (end 87.1 115.3) (width 0.57) (layer "F.Cu") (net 18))
 (segment (start 66.96211 127.439998) (end 58.622112 119.1) (width 0.57) (layer "F.Cu") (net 18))
 (segment (start 51.1 119.1) (end 49 117) (width 0.57) (layer "F.Cu") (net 18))
 (segment (start 99.069999 128.600945) (end 97.830946 129.839998) (width 0.57) (layer "F.Cu") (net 18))
 (segment (start 98.3 118.9) (end 98.3 128.282) (width 0.57) (layer "F.Cu") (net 19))
 (segment (start 58.911056 118.3) (end 52.4 118.3) (width 0.57) (layer "F.Cu") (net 19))
 (segment (start 86.781055 116.069999) (end 95.47 116.07) (width 0.57) (layer "F.Cu") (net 19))
 (segment (start 85.24755 114.536494) (end 86.781055 116.069999) (width 0.57) (layer "F.Cu") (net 19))
 (segment (start 70.37 126.67) (end 67.281055 126.669999) (width 0.57) (layer "F.Cu") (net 19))
 (segment (start 85.24755 113.5695) (end 85.24755 114.536494) (width 0.57) (layer "F.Cu") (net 19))
 (segment (start 52.4 118.3) (end 51 116.9) (width 0.57) (layer "F.Cu") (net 19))
 (segment (start 72.769999 129.069999) (end 70.37 126.67) (width 0.57) (layer "F.Cu") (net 19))
 (segment (start 98.3 128.282) (end 97.512001 129.069999) (width 0.57) (layer "F.Cu") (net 19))
 (segment (start 67.281055 126.669999) (end 58.911056 118.3) (width 0.57) (layer "F.Cu") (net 19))
 (segment (start 95.47 116.07) (end 98.3 118.9) (width 0.57) (layer "F.Cu") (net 19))
 (segment (start 51 116.9) (end 51 112.5) (width 0.57) (layer "F.Cu") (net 19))
 (segment (start 97.512001 129.069999) (end 72.769999 129.069999) (width 0.57) (layer "F.Cu") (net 19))
 (segment (start 70.28 120) (end 64.966832 120) (width 0.57) (layer "F.Cu") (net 9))
 (segment (start 59.8 114.833168) (end 59.8 107.7) (width 0.57) (layer "F.Cu") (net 9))
 (segment (start 59.8 107.7) (end 61 106.5) (width 0.57) (layer "F.Cu") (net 9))
 (segment (start 64.966832 120) (end 59.8 114.833168) (width 0.57) (layer "F.Cu") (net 9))
 (segment (start 61.1 106.5) (end 61 106.5) (width 0.25) (layer "F.Cu") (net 9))
 (segment (start 71.7 113.1) (end 72.492435 112.307565) (width 0.57) (layer "F.Cu") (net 10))
 (segment (start 65.98 115.3) (end 68.18 113.1) (width 0.57) (layer "F.Cu") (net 10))
 (segment (start 68.18 113.1) (end 71.7 113.1) (width 0.57) (layer "F.Cu") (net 10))
 (segment (start 72.492435 112.307565) (end 72.492435 107.192435) (width 0.57) (layer "F.Cu") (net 10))
 (segment (start 72.492435 107.192435) (end 71.8 106.5) (width 0.57) (layer "F.Cu") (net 10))
 (segment (start 71.8 106.5) (end 71 106.5) (width 0.57) (layer "F.Cu") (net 10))
 (segment (start 53 112.5) (end 53 114.58) (width 0.57) (layer "F.Cu") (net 21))
 (segment (start 55 112.5) (end 55 114.58) (width 0.57) (layer "F.Cu") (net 2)))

